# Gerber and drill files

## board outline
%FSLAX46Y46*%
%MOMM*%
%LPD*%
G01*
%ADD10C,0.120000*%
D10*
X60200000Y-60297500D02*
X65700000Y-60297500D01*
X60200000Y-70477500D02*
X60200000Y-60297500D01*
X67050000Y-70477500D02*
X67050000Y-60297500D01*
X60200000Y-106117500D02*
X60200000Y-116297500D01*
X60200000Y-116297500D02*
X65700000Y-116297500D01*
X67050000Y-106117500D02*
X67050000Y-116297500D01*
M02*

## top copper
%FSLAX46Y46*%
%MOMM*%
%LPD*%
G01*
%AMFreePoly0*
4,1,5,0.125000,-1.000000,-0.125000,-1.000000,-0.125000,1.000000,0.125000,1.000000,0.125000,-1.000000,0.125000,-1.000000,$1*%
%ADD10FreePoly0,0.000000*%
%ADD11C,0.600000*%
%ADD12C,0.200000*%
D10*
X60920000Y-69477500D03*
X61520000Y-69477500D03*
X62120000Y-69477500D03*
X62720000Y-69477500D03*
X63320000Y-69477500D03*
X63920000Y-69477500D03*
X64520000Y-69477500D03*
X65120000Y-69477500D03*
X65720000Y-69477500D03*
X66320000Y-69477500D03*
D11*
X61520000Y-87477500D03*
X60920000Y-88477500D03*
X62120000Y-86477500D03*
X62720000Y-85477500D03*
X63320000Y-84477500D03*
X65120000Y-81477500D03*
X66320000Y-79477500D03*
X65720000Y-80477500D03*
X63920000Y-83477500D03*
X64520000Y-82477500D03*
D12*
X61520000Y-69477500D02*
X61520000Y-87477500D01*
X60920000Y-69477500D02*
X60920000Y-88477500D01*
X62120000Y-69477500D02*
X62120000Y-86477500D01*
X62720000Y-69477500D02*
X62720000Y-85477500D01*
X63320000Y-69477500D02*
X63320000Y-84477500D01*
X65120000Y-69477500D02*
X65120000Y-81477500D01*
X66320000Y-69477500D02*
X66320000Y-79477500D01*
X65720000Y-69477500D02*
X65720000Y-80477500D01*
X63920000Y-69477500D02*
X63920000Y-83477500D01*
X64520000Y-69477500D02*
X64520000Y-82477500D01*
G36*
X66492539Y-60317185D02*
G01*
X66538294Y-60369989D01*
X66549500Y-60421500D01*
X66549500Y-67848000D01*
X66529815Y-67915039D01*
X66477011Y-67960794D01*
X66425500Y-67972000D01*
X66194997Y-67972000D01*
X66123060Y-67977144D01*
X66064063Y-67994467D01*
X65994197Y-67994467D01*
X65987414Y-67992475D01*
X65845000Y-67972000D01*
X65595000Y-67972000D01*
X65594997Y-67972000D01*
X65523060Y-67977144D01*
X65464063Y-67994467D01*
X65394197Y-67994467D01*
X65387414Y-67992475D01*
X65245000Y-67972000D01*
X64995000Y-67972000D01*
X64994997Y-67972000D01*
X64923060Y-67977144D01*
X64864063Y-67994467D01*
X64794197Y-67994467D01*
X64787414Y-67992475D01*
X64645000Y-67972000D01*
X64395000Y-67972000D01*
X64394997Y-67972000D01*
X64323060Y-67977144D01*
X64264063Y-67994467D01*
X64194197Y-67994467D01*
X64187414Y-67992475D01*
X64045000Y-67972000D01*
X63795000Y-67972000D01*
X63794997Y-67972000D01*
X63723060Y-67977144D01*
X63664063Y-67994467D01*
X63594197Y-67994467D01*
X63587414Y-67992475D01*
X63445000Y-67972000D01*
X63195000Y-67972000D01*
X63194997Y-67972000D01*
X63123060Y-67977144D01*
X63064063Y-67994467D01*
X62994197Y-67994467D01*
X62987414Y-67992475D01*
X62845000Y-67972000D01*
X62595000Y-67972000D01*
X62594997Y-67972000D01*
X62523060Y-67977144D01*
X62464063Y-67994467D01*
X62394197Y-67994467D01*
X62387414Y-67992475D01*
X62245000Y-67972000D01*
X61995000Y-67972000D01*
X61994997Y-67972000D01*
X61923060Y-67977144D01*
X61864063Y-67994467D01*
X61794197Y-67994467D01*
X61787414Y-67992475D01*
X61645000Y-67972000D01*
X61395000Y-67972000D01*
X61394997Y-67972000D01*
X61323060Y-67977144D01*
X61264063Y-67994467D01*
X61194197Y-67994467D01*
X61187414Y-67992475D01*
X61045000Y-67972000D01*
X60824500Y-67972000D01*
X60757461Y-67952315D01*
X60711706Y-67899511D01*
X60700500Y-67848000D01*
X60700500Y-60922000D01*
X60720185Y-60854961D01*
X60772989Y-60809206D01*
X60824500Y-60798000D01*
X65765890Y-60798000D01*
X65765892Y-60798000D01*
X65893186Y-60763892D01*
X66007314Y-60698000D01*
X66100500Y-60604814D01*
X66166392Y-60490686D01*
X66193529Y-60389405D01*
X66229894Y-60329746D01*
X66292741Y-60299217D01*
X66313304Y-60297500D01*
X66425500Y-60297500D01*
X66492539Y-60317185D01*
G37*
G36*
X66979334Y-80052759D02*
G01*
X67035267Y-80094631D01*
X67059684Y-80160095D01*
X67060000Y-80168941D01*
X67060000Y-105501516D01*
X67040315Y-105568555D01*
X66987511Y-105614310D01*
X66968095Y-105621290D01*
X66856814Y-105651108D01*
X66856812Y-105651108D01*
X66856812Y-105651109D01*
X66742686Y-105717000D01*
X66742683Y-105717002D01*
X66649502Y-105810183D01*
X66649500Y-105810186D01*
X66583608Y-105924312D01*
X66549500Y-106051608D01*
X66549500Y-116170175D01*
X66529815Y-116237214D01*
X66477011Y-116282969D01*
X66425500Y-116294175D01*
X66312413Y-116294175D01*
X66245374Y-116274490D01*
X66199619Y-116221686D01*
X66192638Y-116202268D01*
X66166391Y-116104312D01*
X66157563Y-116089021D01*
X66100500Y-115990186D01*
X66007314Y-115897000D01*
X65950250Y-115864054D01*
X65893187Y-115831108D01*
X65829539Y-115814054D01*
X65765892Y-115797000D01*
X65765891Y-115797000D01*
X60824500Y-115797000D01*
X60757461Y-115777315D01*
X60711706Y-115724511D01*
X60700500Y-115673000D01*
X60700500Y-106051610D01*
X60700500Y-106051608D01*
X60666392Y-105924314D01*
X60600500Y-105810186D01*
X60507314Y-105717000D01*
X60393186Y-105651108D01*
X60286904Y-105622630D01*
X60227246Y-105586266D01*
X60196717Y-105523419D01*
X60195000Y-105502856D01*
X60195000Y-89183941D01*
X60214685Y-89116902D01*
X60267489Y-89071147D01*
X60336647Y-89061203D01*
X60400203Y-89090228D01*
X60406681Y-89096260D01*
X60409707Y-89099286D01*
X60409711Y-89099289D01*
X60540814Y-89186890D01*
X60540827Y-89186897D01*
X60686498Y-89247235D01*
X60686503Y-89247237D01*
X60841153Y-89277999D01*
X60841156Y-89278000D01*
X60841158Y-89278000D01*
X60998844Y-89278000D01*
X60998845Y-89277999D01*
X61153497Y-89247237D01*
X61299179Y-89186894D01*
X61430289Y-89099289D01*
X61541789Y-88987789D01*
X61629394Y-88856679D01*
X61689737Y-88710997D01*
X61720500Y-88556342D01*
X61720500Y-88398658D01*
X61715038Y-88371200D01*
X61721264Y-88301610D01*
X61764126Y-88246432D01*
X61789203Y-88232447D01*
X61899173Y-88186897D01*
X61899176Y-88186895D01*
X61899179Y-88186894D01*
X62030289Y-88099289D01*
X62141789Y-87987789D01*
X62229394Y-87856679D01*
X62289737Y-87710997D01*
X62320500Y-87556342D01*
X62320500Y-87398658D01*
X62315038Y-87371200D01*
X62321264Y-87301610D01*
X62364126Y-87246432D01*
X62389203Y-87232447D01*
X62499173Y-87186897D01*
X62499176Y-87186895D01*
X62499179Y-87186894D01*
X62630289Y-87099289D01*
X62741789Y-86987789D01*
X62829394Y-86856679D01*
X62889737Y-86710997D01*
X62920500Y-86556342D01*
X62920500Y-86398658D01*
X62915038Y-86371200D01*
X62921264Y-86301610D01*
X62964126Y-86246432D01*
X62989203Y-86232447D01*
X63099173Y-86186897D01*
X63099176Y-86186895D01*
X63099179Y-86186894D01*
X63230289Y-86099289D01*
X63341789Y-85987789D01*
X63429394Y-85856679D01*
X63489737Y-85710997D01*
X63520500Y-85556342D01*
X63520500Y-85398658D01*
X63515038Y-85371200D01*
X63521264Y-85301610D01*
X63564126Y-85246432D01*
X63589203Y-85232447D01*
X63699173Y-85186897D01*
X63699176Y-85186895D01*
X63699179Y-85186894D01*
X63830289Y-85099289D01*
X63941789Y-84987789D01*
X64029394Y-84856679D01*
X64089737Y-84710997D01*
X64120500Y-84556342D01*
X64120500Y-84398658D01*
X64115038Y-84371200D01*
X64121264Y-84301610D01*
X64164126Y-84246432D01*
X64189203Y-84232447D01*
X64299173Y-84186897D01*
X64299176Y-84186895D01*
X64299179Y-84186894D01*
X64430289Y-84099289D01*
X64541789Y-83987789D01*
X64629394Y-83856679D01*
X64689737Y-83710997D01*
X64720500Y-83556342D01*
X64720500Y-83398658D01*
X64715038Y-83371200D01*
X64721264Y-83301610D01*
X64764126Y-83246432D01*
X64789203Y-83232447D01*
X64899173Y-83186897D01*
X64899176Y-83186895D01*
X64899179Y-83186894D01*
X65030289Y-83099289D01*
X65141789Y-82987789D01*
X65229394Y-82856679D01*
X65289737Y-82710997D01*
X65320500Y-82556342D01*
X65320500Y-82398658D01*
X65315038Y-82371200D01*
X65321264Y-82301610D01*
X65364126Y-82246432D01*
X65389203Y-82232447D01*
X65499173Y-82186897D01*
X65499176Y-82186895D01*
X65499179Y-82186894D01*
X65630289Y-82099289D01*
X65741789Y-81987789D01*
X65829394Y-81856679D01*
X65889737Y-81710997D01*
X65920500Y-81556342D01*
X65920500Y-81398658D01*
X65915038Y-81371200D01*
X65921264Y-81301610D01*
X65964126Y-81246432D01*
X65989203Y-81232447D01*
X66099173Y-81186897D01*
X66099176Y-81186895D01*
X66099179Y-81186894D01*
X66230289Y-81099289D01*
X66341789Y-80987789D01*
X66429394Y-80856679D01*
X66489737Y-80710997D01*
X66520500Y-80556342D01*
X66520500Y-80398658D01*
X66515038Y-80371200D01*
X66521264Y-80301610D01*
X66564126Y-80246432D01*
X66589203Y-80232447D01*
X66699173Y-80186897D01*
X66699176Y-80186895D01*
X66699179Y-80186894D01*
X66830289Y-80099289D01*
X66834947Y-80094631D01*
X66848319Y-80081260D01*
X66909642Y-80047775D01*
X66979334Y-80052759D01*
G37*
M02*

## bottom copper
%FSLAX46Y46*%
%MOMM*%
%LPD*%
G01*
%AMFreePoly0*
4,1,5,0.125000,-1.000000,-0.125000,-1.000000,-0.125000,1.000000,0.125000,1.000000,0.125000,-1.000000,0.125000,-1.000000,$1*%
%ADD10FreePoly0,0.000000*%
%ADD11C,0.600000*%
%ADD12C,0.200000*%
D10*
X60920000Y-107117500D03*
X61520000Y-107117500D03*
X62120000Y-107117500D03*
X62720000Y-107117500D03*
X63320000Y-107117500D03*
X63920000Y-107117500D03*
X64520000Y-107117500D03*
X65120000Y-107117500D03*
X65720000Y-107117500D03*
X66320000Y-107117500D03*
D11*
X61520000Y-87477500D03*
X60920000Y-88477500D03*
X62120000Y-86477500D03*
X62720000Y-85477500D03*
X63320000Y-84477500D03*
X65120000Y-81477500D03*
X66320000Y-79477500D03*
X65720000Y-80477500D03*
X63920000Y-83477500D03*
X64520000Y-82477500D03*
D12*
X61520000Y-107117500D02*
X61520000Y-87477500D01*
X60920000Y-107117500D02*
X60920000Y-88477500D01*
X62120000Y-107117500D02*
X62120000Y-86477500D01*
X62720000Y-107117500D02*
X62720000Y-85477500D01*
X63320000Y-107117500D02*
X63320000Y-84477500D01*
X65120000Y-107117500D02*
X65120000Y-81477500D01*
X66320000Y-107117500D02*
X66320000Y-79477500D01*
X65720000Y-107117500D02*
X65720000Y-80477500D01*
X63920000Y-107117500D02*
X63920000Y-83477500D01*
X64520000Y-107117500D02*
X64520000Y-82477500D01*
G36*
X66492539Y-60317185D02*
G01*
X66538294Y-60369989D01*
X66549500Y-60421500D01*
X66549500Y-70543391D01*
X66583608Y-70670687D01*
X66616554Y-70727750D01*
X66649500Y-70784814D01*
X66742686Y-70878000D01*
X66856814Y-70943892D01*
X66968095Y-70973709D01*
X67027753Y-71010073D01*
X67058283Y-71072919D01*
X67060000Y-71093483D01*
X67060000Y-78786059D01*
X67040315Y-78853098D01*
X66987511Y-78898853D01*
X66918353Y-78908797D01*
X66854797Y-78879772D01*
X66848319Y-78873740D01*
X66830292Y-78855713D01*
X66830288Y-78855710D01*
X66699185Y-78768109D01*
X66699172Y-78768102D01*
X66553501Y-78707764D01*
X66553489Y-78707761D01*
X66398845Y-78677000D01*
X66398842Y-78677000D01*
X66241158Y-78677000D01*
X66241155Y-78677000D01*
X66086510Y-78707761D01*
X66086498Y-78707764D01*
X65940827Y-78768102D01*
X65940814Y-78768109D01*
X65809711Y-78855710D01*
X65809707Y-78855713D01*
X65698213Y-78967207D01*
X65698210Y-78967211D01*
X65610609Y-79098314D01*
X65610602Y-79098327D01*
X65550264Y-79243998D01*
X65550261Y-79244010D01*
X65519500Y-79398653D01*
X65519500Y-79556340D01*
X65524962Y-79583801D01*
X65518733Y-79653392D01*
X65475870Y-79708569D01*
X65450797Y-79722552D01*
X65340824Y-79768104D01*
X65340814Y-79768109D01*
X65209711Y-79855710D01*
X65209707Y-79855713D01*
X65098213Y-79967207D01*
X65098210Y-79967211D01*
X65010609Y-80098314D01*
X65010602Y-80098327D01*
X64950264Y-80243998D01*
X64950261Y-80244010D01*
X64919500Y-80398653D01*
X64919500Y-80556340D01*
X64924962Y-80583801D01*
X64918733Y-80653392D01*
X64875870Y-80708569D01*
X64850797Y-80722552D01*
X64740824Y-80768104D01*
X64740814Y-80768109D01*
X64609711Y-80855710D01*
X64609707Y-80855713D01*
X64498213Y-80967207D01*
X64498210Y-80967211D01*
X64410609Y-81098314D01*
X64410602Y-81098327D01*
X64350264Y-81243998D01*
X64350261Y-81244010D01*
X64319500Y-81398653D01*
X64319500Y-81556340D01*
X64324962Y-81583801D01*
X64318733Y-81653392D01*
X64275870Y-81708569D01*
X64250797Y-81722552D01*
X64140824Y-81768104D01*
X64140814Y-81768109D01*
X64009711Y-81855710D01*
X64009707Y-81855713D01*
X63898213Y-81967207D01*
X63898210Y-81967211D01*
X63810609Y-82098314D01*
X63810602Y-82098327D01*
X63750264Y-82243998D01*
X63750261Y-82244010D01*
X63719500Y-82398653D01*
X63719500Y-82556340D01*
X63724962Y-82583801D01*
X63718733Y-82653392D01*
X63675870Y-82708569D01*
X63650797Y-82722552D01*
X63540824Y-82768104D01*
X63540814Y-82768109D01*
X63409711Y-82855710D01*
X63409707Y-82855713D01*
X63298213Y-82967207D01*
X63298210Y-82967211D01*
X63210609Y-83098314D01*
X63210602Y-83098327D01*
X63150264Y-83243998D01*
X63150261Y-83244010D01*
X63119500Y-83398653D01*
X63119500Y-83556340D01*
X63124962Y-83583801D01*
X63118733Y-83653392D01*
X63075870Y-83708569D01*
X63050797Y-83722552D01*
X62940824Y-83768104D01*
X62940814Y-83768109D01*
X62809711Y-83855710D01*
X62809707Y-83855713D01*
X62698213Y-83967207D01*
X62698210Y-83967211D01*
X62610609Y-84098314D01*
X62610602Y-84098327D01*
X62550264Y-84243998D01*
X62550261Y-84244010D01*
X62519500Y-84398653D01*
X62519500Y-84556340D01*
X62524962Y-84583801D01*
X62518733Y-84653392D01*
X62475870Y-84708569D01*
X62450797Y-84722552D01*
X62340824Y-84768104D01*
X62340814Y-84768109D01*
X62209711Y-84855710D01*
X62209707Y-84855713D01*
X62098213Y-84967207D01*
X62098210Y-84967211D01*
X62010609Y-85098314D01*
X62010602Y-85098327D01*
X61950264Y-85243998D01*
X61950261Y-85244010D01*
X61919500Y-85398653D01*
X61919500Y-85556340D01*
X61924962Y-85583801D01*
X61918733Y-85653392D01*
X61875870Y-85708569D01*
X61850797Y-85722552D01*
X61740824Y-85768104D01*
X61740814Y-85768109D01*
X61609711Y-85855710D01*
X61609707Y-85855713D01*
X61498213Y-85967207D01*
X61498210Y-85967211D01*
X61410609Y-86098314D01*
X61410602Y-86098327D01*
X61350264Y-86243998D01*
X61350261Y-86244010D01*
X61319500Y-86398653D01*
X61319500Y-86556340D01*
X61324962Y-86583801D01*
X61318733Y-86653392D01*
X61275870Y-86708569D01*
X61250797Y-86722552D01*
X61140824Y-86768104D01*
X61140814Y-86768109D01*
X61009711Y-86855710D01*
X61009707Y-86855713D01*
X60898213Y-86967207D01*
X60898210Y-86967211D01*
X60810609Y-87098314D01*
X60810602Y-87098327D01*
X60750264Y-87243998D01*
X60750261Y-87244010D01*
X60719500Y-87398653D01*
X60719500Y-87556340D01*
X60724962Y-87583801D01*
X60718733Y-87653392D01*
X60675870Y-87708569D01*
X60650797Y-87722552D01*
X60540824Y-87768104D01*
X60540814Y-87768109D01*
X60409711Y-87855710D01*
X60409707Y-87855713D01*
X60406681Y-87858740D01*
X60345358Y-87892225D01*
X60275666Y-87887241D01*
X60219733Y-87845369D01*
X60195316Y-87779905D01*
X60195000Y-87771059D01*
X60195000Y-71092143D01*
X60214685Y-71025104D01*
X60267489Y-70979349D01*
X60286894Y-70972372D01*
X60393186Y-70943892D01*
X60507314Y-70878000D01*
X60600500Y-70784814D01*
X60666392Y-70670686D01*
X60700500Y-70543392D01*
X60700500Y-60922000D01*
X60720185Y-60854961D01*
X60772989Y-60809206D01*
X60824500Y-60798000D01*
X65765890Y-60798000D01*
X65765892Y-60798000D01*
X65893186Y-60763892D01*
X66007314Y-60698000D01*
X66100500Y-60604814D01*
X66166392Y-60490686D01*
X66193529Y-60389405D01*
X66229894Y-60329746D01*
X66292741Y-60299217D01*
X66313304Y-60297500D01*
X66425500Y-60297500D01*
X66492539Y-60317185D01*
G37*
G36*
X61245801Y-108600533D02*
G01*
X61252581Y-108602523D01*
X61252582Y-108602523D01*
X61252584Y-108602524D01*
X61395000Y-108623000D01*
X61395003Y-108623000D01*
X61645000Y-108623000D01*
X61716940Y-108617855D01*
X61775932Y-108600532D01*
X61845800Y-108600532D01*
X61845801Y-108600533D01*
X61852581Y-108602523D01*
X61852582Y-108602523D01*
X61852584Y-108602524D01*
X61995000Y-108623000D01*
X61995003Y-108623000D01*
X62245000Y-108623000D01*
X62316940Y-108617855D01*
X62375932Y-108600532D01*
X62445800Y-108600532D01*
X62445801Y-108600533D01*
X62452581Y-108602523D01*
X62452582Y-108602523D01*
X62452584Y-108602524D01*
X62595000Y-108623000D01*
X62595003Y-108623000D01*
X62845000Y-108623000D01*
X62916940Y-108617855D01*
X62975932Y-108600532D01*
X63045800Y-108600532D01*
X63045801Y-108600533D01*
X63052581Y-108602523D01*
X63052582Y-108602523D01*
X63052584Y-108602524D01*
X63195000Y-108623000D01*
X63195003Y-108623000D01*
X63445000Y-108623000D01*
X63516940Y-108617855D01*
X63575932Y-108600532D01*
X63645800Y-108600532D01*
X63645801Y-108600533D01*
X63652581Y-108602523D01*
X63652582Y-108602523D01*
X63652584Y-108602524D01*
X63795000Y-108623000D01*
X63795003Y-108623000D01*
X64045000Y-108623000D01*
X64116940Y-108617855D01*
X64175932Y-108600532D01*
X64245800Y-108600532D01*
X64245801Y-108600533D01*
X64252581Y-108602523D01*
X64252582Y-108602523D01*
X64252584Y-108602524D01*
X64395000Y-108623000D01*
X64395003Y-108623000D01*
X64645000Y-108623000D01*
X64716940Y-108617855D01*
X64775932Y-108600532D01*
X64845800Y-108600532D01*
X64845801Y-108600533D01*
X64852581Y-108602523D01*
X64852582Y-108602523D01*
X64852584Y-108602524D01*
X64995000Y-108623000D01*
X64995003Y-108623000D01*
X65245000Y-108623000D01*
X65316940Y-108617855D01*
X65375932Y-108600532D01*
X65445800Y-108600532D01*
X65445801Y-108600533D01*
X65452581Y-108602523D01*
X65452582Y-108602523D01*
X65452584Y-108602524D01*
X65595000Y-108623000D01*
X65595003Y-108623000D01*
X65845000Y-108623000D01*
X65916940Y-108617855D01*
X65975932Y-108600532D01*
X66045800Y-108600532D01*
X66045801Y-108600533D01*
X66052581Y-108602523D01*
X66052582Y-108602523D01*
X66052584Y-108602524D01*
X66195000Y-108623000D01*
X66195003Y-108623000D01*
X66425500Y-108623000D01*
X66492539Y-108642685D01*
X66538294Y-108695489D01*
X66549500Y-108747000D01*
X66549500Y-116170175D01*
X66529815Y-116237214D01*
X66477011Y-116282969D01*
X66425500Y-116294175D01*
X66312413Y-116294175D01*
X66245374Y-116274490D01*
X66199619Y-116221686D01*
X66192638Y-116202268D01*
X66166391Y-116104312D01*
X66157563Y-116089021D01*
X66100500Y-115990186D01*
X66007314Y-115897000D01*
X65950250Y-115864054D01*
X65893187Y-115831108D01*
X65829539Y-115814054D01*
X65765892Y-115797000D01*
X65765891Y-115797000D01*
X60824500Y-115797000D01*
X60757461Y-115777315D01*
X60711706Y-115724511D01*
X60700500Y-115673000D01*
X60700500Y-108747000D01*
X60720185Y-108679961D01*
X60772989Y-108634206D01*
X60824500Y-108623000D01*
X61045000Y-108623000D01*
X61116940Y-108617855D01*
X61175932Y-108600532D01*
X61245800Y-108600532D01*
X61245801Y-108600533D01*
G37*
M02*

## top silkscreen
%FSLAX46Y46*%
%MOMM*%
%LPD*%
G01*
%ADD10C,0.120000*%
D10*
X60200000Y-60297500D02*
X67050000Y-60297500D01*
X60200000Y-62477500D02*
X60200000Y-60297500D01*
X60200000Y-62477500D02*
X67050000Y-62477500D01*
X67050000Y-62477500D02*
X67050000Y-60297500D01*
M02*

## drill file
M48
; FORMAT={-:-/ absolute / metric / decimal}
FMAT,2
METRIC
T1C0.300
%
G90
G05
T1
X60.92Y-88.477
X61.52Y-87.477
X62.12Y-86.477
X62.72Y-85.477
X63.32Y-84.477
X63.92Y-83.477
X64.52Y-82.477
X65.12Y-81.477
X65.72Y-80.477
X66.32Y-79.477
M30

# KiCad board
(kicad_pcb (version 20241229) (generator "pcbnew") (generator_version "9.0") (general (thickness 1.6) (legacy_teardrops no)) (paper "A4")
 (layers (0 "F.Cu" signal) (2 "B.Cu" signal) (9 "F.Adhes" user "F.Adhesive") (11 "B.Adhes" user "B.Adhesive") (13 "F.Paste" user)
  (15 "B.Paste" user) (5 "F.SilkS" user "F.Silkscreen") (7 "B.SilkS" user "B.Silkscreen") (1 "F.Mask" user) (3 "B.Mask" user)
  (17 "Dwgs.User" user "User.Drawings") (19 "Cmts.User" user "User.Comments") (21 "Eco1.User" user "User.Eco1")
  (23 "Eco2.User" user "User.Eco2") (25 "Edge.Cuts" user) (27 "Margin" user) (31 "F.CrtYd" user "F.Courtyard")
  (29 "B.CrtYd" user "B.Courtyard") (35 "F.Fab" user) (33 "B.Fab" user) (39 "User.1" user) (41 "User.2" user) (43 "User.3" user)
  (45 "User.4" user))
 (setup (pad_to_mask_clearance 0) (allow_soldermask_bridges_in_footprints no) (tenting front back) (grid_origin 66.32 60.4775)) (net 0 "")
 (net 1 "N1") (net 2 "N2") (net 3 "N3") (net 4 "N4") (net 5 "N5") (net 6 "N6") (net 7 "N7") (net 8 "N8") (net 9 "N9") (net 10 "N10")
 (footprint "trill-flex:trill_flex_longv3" (layer "F.Cu") (at 68.45 62.4775)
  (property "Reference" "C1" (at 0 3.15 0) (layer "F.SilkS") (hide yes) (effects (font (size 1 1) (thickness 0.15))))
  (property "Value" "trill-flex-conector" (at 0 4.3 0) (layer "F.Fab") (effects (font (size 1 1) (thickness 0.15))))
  (fp_line (start -8.25 -2.18) (end -1.4 -2.18) (stroke (width 0.12) (type solid)) (layer "F.SilkS"))
  (fp_line (start -8.25 0) (end -8.25 -2.18) (stroke (width 0.12) (type solid)) (layer "F.SilkS"))
  (fp_line (start -8.25 0) (end -1.4 0) (stroke (width 0.12) (type solid)) (layer "F.SilkS"))
  (fp_line (start -1.4 0) (end -1.4 -2.18) (stroke (width 0.12) (type solid)) (layer "F.SilkS"))
  (fp_line (start -8.25 -2.18) (end -2.75 -2.18) (stroke (width 0.12) (type solid)) (layer "Edge.Cuts"))
  (fp_line (start -8.25 8) (end -8.25 -2.18) (stroke (width 0.12) (type solid)) (layer "Edge.Cuts"))
  (fp_line (start -1.4 8) (end -1.4 -2.18) (stroke (width 0.12) (type solid)) (layer "Edge.Cuts"))
  (pad "" smd rect (at -7.53 0) (size 0.25 4) (layers "F.Mask" "F.Paste"))
  (pad "" smd rect (at -6.93 0) (size 0.25 4) (layers "F.Mask" "F.Paste"))
  (pad "" smd rect (at -6.33 0) (size 0.25 4) (layers "F.Mask" "F.Paste"))
  (pad "" smd rect (at -5.73 0) (size 0.25 4) (layers "F.Mask" "F.Paste"))
  (pad "" smd rect (at -5.13 0) (size 0.25 4) (layers "F.Mask" "F.Paste"))
  (pad "" smd rect (at -4.53 0) (size 0.25 4) (layers "F.Mask" "F.Paste"))
  (pad "" smd rect (at -3.93 0) (size 0.25 4) (layers "F.Mask" "F.Paste"))
  (pad "" smd rect (at -3.33 0) (size 0.25 4) (layers "F.Mask" "F.Paste"))
  (pad "" smd rect (at -2.73 0) (size 0.25 4) (layers "F.Mask" "F.Paste"))
  (pad "" smd rect (at -2.13 0) (size 0.25 4) (layers "F.Mask" "F.Paste"))
  (pad "1" smd custom (at -7.53 7) (size 0.25 2) (layers "F.Cu") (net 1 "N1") (zone_connect 0) (options (clearance outline) (anchor rect))
   (primitives))
  (pad "2" smd custom (at -6.93 7) (size 0.25 2) (layers "F.Cu") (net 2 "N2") (zone_connect 0) (options (clearance outline) (anchor rect))
   (primitives))
  (pad "3" smd custom (at -6.33 7) (size 0.25 2) (layers "F.Cu") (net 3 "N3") (zone_connect 0) (options (clearance outline) (anchor rect))
   (primitives))
  (pad "4" smd custom (at -5.73 7) (size 0.25 2) (layers "F.Cu") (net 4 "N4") (zone_connect 0) (options (clearance outline) (anchor rect))
   (primitives))
  (pad "5" smd custom (at -5.13 7) (size 0.25 2) (layers "F.Cu") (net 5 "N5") (zone_connect 0) (options (clearance outline) (anchor rect))
   (primitives))
  (pad "6" smd custom (at -4.53 7) (size 0.25 2) (layers "F.Cu") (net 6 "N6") (zone_connect 0) (options (clearance outline) (anchor rect))
   (primitives))
  (pad "7" smd custom (at -3.93 7) (size 0.25 2) (layers "F.Cu") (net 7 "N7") (zone_connect 0) (options (clearance outline) (anchor rect))
   (primitives))
  (pad "8" smd custom (at -3.33 7) (size 0.25 2) (layers "F.Cu") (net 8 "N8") (zone_connect 0) (options (clearance outline) (anchor rect))
   (primitives))
  (pad "9" smd custom (at -2.73 7) (size 0.25 2) (layers "F.Cu") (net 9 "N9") (zone_connect 0) (options (clearance outline) (anchor rect))
   (primitives))
  (pad "10" smd custom (at -2.13 7) (size 0.25 2) (layers "F.Cu") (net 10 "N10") (zone_connect 0)
   (options (clearance outline) (anchor rect)) (primitives)))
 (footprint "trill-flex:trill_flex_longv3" (layer "B.Cu") (at 68.45 114.1175)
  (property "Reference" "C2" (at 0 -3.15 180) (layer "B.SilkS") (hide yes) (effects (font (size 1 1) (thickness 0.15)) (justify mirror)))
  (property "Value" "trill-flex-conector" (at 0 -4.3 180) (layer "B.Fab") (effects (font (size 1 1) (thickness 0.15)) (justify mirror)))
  (fp_line (start -8.25 -8) (end -8.25 2.18) (stroke (width 0.12) (type solid)) (layer "Edge.Cuts"))
  (fp_line (start -8.25 2.18) (end -2.75 2.18) (stroke (width 0.12) (type solid)) (layer "Edge.Cuts"))
  (fp_line (start -1.4 -8) (end -1.4 2.18) (stroke (width 0.12) (type solid)) (layer "Edge.Cuts"))
  (pad "" smd rect (at -7.53 0) (size 0.25 4) (layers "B.Mask" "B.Paste"))
  (pad "" smd rect (at -6.93 0) (size 0.25 4) (layers "B.Mask" "B.Paste"))
  (pad "" smd rect (at -6.33 0) (size 0.25 4) (layers "B.Mask" "B.Paste"))
  (pad "" smd rect (at -5.73 0) (size 0.25 4) (layers "B.Mask" "B.Paste"))
  (pad "" smd rect (at -5.13 0) (size 0.25 4) (layers "B.Mask" "B.Paste"))
  (pad "" smd rect (at -4.53 0) (size 0.25 4) (layers "B.Mask" "B.Paste"))
  (pad "" smd rect (at -3.93 0) (size 0.25 4) (layers "B.Mask" "B.Paste"))
  (pad "" smd rect (at -3.33 0) (size 0.25 4) (layers "B.Mask" "B.Paste"))
  (pad "" smd rect (at -2.73 0) (size 0.25 4) (layers "B.Mask" "B.Paste"))
  (pad "" smd rect (at -2.13 0) (size 0.25 4) (layers "B.Mask" "B.Paste"))
  (pad "1" smd custom (at -7.53 -7) (size 0.25 2) (layers "B.Cu") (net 1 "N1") (zone_connect 0) (options (clearance outline) (anchor rect))
   (primitives))
  (pad "2" smd custom (at -6.93 -7) (size 0.25 2) (layers "B.Cu") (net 2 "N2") (zone_connect 0) (options (clearance outline) (anchor rect))
   (primitives))
  (pad "3" smd custom (at -6.33 -7) (size 0.25 2) (layers "B.Cu") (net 3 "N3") (zone_connect 0) (options (clearance outline) (anchor rect))
   (primitives))
  (pad "4" smd custom (at -5.73 -7) (size 0.25 2) (layers "B.Cu") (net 4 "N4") (zone_connect 0) (options (clearance outline) (anchor rect))
   (primitives))
  (pad "5" smd custom (at -5.13 -7) (size 0.25 2) (layers "B.Cu") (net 5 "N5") (zone_connect 0) (options (clearance outline) (anchor rect))
   (primitives))
  (pad "6" smd custom (at -4.53 -7) (size 0.25 2) (layers "B.Cu") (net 6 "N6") (zone_connect 0) (options (clearance outline) (anchor rect))
   (primitives))
  (pad "7" smd custom (at -3.93 -7) (size 0.25 2) (layers "B.Cu") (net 7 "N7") (zone_connect 0) (options (clearance outline) (anchor rect))
   (primitives))
  (pad "8" smd custom (at -3.33 -7) (size 0.25 2) (layers "B.Cu") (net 8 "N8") (zone_connect 0) (options (clearance outline) (anchor rect))
   (primitives))
  (pad "9" smd custom (at -2.73 -7) (size 0.25 2) (layers "B.Cu") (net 9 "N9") (zone_connect 0) (options (clearance outline) (anchor rect))
   (primitives))
  (pad "10" smd custom (at -2.13 -7) (size 0.25 2) (layers "B.Cu") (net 10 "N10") (zone_connect 0)
   (options (clearance outline) (anchor rect)) (primitives)))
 (segment (start 61.52 69.4775) (end 61.52 87.4775) (width 0.2) (layer "F.Cu") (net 2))
 (via (at 61.52 87.4775) (size 0.6) (drill 0.3) (layers "F.Cu" "B.Cu") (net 2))
 (segment (start 61.52 107.1175) (end 61.52 87.4775) (width 0.2) (layer "B.Cu") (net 2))
 (segment (start 60.92 69.4775) (end 60.92 88.4775) (width 0.2) (layer "F.Cu") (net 1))
 (via (at 60.92 88.4775) (size 0.6) (drill 0.3) (layers "F.Cu" "B.Cu") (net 1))
 (segment (start 60.92 107.1175) (end 60.92 88.4775) (width 0.2) (layer "B.Cu") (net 1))
 (segment (start 62.12 69.4775) (end 62.12 86.4775) (width 0.2) (layer "F.Cu") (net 3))
 (via (at 62.12 86.4775) (size 0.6) (drill 0.3) (layers "F.Cu" "B.Cu") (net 3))
 (segment (start 62.12 107.1175) (end 62.12 86.4775) (width 0.2) (layer "B.Cu") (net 3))
 (segment (start 62.72 69.4775) (end 62.72 85.4775) (width 0.2) (layer "F.Cu") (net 4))
 (via (at 62.72 85.4775) (size 0.6) (drill 0.3) (layers "F.Cu" "B.Cu") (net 4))
 (segment (start 62.72 107.1175) (end 62.72 85.4775) (width 0.2) (layer "B.Cu") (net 4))
 (segment (start 63.32 69.4775) (end 63.32 84.4775) (width 0.2) (layer "F.Cu") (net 5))
 (via (at 63.32 84.4775) (size 0.6) (drill 0.3) (layers "F.Cu" "B.Cu") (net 5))
 (segment (start 63.32 107.1175) (end 63.32 84.4775) (width 0.2) (layer "B.Cu") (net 5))
 (segment (start 65.12 69.4775) (end 65.12 81.4775) (width 0.2) (layer "F.Cu") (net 8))
 (via (at 65.12 81.4775) (size 0.6) (drill 0.3) (layers "F.Cu" "B.Cu") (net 8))
 (segment (start 65.12 107.1175) (end 65.12 81.4775) (width 0.2) (layer "B.Cu") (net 8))
 (segment (start 66.32 69.4775) (end 66.32 79.4775) (width 0.2) (layer "F.Cu") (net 10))
 (via (at 66.32 79.4775) (size 0.6) (drill 0.3) (layers "F.Cu" "B.Cu") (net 10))
 (segment (start 66.32 107.1175) (end 66.32 79.4775) (width 0.2) (layer "B.Cu") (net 10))
 (segment (start 65.72 69.4775) (end 65.72 80.4775) (width 0.2) (layer "F.Cu") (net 9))
 (via (at 65.72 80.4775) (size 0.6) (drill 0.3) (layers "F.Cu" "B.Cu") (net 9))
 (segment (start 65.72 107.1175) (end 65.72 80.4775) (width 0.2) (layer "B.Cu") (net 9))
 (segment (start 63.92 69.4775) (end 63.92 83.4775) (width 0.2) (layer "F.Cu") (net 6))
 (via (at 63.92 83.4775) (size 0.6) (drill 0.3) (layers "F.Cu" "B.Cu") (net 6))
 (segment (start 63.92 107.1175) (end 63.92 83.4775) (width 0.2) (layer "B.Cu") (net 6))
 (segment (start 64.52 69.4775) (end 64.52 82.4775) (width 0.2) (layer "F.Cu") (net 7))
 (via (at 64.52 82.4775) (size 0.6) (drill 0.3) (layers "F.Cu" "B.Cu") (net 7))
 (segment (start 64.52 107.1175) (end 64.52 82.4775) (width 0.2) (layer "B.Cu") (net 7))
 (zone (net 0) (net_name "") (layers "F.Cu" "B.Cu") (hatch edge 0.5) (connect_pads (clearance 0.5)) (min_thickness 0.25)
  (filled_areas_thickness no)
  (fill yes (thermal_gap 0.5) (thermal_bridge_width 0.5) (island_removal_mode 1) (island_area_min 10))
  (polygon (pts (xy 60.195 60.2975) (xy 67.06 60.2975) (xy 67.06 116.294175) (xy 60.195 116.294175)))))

